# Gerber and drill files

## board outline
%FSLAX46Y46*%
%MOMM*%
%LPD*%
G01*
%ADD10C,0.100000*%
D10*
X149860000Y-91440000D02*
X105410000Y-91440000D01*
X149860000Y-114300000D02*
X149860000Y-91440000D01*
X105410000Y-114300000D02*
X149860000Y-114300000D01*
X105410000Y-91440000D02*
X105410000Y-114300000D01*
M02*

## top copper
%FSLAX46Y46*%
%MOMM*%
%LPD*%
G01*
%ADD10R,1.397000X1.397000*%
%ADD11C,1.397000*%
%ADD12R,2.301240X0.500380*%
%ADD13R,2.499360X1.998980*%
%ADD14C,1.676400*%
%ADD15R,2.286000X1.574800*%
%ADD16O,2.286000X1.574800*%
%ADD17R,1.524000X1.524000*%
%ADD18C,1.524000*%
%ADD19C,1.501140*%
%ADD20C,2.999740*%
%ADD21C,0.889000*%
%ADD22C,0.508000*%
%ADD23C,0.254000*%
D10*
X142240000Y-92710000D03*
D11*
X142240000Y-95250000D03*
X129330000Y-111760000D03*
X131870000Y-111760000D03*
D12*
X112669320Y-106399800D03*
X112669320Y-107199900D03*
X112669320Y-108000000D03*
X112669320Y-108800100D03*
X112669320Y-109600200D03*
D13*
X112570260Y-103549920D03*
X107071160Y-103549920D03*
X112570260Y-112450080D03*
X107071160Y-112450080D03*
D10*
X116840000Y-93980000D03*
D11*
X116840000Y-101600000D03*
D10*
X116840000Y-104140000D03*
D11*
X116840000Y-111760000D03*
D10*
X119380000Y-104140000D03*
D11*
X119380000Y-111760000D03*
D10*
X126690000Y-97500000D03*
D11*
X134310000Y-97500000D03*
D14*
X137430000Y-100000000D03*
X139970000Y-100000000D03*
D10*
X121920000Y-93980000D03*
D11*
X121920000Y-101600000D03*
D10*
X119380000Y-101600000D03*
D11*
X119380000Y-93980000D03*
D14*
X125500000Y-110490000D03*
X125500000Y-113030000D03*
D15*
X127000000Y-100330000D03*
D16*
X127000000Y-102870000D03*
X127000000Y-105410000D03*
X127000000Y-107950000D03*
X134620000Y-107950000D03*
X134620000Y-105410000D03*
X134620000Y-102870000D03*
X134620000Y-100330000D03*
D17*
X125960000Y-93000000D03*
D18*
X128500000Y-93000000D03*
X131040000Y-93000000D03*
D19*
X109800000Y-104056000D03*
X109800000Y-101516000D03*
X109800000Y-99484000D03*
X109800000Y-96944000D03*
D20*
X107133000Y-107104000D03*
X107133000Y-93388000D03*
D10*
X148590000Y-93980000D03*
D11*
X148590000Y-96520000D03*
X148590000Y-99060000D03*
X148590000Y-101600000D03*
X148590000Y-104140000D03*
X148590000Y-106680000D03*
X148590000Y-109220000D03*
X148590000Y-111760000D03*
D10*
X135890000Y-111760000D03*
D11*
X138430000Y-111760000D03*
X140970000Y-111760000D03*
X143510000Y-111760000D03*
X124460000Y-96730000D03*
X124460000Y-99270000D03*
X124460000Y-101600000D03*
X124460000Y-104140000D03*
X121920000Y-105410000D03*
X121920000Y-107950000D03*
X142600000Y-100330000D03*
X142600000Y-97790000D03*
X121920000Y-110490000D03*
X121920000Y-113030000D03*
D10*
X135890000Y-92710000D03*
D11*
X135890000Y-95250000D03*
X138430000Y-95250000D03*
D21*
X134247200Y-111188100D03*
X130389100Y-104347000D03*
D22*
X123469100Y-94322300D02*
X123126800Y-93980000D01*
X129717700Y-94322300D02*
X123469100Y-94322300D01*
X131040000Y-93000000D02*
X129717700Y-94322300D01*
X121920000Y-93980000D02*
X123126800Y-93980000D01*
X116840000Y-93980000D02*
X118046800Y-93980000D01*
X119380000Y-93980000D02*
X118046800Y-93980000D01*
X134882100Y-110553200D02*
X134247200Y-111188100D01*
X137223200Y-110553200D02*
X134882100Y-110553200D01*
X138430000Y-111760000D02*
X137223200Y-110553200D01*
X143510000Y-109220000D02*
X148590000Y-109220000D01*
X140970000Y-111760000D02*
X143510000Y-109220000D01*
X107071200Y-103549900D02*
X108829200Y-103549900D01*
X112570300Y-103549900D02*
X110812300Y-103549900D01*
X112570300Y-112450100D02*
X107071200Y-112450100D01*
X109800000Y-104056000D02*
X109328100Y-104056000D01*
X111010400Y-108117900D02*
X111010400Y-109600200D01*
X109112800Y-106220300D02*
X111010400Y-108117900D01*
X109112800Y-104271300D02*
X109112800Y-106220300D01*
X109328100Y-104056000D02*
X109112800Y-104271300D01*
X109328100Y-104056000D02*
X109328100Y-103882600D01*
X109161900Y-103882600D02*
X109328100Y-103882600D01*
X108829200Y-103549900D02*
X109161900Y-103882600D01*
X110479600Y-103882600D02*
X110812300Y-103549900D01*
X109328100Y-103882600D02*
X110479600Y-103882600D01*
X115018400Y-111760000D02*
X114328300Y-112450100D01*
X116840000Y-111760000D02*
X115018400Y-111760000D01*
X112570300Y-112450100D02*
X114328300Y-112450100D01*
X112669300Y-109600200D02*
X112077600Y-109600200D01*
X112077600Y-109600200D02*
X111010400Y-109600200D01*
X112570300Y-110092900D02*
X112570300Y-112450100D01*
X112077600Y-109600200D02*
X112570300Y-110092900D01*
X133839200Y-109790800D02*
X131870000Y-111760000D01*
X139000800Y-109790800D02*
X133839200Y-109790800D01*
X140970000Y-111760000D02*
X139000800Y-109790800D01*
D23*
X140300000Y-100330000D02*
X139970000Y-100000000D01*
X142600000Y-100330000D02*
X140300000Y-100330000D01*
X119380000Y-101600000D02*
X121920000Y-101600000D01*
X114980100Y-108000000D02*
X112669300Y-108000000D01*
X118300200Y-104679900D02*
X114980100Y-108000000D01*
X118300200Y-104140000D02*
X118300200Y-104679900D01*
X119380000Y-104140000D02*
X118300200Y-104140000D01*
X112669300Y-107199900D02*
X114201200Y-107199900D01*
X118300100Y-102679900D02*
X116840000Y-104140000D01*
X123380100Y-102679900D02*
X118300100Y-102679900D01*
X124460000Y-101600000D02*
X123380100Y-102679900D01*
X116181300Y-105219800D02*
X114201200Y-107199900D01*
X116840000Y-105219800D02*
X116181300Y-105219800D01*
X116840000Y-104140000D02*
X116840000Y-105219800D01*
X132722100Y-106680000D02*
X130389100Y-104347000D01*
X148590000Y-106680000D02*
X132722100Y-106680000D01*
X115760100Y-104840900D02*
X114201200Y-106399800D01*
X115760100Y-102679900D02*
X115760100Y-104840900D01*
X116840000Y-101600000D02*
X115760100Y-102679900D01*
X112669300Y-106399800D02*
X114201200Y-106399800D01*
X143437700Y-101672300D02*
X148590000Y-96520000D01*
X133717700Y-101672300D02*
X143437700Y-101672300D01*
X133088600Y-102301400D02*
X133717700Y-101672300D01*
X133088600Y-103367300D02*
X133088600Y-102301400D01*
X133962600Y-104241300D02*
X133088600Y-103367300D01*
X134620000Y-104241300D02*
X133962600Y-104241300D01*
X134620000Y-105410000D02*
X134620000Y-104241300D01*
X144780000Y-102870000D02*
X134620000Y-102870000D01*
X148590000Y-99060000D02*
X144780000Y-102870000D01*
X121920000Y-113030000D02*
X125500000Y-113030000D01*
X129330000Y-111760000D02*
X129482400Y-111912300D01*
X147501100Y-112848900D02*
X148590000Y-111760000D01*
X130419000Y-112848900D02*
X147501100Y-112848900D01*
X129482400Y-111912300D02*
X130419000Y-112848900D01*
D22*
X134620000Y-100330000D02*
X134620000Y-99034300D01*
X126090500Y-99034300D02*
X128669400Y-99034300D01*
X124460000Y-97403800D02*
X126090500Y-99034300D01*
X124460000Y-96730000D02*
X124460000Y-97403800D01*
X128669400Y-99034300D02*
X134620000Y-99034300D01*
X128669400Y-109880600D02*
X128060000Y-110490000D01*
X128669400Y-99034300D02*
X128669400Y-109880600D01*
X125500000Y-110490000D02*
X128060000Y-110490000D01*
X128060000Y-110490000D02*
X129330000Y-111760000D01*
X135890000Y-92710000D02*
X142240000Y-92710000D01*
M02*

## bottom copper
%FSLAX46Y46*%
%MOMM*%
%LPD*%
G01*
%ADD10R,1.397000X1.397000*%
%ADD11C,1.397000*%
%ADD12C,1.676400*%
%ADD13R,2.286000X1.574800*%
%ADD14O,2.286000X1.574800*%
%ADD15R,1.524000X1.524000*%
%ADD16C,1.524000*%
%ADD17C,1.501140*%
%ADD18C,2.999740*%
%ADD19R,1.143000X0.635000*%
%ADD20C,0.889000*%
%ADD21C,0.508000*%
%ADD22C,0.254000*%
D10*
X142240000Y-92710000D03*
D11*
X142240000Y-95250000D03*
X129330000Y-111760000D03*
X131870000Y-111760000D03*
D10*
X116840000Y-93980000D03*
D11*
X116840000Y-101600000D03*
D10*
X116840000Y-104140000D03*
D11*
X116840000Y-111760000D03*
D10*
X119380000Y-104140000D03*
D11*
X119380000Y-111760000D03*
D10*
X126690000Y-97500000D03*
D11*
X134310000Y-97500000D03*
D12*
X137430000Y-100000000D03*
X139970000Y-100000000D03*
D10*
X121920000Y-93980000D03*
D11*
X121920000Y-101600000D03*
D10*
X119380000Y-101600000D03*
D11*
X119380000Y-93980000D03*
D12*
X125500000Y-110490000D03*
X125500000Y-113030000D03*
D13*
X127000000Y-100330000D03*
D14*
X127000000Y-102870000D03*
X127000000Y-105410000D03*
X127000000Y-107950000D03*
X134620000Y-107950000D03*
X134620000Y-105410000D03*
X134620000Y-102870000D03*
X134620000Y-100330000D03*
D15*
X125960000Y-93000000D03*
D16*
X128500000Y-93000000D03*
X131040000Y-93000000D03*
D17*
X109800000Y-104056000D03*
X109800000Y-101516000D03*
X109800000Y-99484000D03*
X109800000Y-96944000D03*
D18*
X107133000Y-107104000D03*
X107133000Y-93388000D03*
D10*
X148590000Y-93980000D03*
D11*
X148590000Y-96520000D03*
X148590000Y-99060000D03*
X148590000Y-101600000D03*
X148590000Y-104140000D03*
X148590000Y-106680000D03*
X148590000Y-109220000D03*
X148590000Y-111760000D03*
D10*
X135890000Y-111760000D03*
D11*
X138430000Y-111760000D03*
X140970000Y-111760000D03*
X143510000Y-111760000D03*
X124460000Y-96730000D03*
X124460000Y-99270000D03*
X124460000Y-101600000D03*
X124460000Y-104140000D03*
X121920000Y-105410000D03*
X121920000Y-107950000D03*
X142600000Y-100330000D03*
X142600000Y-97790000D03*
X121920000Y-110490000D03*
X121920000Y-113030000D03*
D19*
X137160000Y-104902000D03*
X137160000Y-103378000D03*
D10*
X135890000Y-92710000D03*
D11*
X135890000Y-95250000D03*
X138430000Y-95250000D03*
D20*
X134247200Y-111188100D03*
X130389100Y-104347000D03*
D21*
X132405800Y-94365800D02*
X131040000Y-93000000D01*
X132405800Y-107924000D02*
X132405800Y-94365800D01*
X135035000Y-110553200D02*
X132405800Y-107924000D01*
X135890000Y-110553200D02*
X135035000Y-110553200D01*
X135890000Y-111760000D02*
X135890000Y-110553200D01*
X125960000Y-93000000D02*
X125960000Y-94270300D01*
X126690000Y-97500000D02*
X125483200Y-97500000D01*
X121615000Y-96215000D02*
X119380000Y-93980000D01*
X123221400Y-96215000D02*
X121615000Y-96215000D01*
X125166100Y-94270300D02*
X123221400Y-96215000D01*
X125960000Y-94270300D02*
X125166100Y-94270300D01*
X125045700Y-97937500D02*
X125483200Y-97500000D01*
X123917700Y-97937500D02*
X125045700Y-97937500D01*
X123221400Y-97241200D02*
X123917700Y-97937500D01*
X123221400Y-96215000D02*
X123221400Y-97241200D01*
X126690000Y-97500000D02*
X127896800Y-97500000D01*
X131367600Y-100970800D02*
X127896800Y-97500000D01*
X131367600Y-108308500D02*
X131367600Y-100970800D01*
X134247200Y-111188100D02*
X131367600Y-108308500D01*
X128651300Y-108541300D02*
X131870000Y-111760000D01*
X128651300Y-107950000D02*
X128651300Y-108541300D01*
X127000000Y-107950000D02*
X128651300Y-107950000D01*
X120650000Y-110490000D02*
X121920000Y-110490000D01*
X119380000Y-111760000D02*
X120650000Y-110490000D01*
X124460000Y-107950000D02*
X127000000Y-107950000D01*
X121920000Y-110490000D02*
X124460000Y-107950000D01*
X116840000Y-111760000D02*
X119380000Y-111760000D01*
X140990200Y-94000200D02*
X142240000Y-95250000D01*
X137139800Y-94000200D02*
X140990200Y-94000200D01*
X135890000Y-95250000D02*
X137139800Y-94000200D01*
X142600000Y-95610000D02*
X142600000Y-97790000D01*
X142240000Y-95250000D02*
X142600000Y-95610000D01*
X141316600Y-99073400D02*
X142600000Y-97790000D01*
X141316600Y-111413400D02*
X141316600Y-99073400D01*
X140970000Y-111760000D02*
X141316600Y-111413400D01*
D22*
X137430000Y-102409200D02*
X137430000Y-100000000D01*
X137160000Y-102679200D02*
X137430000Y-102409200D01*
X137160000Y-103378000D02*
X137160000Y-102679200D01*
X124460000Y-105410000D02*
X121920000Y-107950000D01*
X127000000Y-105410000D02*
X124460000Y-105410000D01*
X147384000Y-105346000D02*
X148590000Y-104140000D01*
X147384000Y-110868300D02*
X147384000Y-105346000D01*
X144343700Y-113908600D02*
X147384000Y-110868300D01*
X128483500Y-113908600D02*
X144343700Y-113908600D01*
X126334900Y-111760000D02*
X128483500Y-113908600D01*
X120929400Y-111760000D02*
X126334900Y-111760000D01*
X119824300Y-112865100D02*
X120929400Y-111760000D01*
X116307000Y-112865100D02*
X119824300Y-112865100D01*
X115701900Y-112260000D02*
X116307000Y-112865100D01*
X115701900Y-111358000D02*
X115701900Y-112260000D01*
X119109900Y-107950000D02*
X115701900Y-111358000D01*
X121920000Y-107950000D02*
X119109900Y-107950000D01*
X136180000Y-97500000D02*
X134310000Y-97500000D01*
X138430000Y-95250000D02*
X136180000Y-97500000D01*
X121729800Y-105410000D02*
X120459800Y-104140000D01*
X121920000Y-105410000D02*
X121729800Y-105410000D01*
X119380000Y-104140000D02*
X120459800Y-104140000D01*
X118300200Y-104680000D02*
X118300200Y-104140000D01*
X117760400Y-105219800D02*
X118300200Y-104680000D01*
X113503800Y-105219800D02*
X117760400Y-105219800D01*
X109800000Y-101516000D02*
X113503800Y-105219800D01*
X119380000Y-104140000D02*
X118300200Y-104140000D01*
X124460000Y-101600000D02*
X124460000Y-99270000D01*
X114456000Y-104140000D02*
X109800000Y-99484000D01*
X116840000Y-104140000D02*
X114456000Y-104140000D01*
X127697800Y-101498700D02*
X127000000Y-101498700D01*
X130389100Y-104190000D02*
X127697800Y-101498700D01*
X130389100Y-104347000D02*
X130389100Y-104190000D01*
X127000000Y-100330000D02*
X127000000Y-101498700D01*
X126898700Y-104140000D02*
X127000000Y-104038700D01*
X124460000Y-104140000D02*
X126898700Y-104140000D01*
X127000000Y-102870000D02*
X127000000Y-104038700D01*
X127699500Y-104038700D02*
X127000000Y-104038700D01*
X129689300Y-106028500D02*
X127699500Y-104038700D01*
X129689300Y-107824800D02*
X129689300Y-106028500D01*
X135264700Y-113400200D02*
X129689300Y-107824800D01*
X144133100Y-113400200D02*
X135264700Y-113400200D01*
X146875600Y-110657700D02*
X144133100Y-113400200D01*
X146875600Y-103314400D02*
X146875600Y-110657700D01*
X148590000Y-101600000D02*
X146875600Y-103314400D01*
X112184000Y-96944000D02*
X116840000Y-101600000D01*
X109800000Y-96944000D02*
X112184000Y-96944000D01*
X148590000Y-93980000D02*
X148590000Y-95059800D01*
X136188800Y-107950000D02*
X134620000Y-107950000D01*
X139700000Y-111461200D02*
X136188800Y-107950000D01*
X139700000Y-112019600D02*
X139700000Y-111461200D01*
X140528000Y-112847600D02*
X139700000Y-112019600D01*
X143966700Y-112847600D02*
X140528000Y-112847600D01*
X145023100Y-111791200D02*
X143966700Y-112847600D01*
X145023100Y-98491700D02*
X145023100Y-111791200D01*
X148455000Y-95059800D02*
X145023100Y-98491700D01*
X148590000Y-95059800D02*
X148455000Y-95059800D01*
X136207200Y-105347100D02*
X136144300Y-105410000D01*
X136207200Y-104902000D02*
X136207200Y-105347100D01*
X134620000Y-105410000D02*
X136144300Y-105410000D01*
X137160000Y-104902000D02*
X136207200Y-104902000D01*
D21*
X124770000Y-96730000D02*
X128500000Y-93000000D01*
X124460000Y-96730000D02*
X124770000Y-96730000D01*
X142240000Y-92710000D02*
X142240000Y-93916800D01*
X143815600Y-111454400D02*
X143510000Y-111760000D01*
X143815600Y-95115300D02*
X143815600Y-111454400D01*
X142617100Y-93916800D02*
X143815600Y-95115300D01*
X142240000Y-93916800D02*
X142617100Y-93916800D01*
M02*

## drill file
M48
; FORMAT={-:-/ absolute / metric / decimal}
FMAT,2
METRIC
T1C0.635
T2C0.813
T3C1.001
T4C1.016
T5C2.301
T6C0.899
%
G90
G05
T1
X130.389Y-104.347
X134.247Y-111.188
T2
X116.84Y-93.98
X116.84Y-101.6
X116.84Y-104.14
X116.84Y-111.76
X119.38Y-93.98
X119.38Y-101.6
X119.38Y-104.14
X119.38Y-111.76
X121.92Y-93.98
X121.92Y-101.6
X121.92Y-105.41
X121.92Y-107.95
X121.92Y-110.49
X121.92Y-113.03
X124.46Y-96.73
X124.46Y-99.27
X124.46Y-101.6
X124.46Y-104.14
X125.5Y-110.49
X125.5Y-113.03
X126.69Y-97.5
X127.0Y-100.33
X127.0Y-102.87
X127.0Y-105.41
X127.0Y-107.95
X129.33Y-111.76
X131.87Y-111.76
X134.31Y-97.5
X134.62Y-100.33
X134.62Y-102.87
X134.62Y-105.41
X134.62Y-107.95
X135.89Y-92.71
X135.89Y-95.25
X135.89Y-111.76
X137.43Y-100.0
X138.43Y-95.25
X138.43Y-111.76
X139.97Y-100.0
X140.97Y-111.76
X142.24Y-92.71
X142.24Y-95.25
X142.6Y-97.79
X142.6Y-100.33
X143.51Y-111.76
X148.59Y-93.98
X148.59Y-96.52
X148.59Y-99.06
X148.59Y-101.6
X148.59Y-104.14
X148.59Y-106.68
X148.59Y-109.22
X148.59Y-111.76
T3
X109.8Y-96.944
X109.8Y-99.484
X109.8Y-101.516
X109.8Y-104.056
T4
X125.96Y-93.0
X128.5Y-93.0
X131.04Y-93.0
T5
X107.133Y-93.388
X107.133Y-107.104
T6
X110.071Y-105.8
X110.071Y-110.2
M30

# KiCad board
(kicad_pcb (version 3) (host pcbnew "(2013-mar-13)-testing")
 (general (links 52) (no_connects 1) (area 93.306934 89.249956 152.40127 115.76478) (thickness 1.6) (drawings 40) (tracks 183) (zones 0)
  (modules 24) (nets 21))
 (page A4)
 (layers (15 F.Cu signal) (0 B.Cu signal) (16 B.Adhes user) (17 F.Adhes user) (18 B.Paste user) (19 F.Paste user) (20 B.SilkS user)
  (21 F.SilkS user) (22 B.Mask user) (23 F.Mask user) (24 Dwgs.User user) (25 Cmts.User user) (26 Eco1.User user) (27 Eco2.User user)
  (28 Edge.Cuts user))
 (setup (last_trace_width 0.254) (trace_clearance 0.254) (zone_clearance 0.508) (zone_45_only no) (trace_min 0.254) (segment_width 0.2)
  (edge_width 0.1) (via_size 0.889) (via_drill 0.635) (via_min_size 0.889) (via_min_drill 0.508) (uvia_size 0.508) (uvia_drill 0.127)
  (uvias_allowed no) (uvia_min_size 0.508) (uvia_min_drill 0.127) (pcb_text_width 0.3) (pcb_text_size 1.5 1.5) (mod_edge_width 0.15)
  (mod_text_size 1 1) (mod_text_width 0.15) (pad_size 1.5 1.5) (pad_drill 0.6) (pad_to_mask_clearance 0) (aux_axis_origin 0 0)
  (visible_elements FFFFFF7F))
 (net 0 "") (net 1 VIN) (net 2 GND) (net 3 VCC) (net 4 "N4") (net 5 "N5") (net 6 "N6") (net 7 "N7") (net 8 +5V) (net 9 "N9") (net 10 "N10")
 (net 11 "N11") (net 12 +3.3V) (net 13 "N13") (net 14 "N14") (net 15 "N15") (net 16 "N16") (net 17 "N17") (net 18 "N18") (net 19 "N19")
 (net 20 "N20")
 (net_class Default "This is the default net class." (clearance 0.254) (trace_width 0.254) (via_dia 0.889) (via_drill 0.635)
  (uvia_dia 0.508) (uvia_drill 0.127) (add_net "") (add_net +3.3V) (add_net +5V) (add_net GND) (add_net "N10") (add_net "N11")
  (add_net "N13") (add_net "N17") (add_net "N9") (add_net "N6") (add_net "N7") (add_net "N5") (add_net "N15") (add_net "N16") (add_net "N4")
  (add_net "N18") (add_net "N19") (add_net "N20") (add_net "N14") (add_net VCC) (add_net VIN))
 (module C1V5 (layer F.Cu) (at 142.24 93.98 270)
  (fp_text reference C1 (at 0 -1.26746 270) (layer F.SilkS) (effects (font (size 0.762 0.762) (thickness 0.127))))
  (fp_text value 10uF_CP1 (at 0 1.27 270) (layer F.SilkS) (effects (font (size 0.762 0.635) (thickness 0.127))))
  (pad 1 thru_hole rect (at -1.27 0 270) (size 1.397 1.397) (drill 0.8128) (layers *.Cu *.Mask F.SilkS) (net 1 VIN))
  (pad 2 thru_hole circle (at 1.27 0 270) (size 1.397 1.397) (drill 0.8128) (layers *.Cu *.Mask F.SilkS) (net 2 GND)))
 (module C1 (layer F.Cu) (at 130.6 111.76)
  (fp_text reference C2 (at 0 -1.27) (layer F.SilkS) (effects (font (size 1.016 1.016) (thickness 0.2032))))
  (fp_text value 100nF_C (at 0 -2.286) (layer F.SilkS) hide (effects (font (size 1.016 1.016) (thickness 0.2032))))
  (pad 1 thru_hole circle (at -1.27 0) (size 1.397 1.397) (drill 0.8128) (layers *.Cu *.Mask F.SilkS) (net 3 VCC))
  (pad 2 thru_hole circle (at 1.27 0) (size 1.397 1.397) (drill 0.8128) (layers *.Cu *.Mask F.SilkS) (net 2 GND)))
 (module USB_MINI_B (layer F.Cu) (at 109.22 108)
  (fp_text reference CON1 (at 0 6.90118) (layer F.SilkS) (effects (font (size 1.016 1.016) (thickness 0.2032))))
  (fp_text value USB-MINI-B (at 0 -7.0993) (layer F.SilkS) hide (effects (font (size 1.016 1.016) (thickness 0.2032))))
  (pad 1 smd rect (at 3.44932 -1.6002) (size 2.30124 0.50038) (layers F.Cu F.Paste F.Mask) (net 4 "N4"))
  (pad 2 smd rect (at 3.44932 -0.8001) (size 2.30124 0.50038) (layers F.Cu F.Paste F.Mask) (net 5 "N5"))
  (pad 3 smd rect (at 3.44932 0) (size 2.30124 0.50038) (layers F.Cu F.Paste F.Mask) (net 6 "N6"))
  (pad 4 smd rect (at 3.44932 0.8001) (size 2.30124 0.50038) (layers F.Cu F.Paste F.Mask) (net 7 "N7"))
  (pad 5 smd rect (at 3.44932 1.6002) (size 2.30124 0.50038) (layers F.Cu F.Paste F.Mask) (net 2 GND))
  (pad 6 smd rect (at 3.35026 -4.45008) (size 2.49936 1.99898) (layers F.Cu F.Paste F.Mask) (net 2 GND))
  (pad 7 smd rect (at -2.14884 -4.45008) (size 2.49936 1.99898) (layers F.Cu F.Paste F.Mask) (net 2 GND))
  (pad 8 smd rect (at 3.35026 4.45008) (size 2.49936 1.99898) (layers F.Cu F.Paste F.Mask) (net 2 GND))
  (pad 9 smd rect (at -2.14884 4.45008) (size 2.49936 1.99898) (layers F.Cu F.Paste F.Mask) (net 2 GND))
  (pad "" np_thru_hole circle (at 0.8509 -2.19964) (size 0.89916 0.89916) (drill 0.89916) (layers *.Cu *.Mask F.SilkS))
  (pad 2 np_thru_hole circle (at 0.8509 2.19964) (size 0.89916 0.89916) (drill 0.89916) (layers *.Cu *.Mask F.SilkS) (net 5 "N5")))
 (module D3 (layer F.Cu) (at 116.84 97.79 90)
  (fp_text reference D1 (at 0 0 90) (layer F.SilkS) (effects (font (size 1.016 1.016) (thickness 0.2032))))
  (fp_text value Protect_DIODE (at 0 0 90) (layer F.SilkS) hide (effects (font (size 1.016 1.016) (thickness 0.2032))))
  (pad 2 thru_hole rect (at 3.81 0 90) (size 1.397 1.397) (drill 0.8128) (layers *.Cu *.Mask F.SilkS) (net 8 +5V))
  (pad 1 thru_hole circle (at -3.81 0 90) (size 1.397 1.397) (drill 0.8128) (layers *.Cu *.Mask F.SilkS) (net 4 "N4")))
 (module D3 (layer F.Cu) (at 116.84 107.95 90)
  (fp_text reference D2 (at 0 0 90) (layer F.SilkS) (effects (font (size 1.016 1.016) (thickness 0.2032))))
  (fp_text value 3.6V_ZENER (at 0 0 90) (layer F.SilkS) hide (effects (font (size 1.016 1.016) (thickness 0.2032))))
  (pad 2 thru_hole rect (at 3.81 0 90) (size 1.397 1.397) (drill 0.8128) (layers *.Cu *.Mask F.SilkS) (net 5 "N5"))
  (pad 1 thru_hole circle (at -3.81 0 90) (size 1.397 1.397) (drill 0.8128) (layers *.Cu *.Mask F.SilkS) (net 2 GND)))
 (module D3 (layer F.Cu) (at 119.38 107.95 90)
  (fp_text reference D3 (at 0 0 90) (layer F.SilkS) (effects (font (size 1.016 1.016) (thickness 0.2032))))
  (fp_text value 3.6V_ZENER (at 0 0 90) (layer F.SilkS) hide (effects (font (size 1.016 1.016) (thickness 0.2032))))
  (pad 2 thru_hole rect (at 3.81 0 90) (size 1.397 1.397) (drill 0.8128) (layers *.Cu *.Mask F.SilkS) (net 6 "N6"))
  (pad 1 thru_hole circle (at -3.81 0 90) (size 1.397 1.397) (drill 0.8128) (layers *.Cu *.Mask F.SilkS) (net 2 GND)))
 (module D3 (layer F.Cu) (at 130.5 97.5 180)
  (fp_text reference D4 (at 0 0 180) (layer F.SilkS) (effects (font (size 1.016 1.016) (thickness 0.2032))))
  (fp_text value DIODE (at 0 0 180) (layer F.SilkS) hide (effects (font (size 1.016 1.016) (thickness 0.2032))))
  (pad 2 thru_hole rect (at 3.81 0 180) (size 1.397 1.397) (drill 0.8128) (layers *.Cu *.Mask F.SilkS) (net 8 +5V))
  (pad 1 thru_hole circle (at -3.81 0 180) (size 1.397 1.397) (drill 0.8128) (layers *.Cu *.Mask F.SilkS) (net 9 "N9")))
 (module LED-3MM (layer F.Cu) (at 138.7 100)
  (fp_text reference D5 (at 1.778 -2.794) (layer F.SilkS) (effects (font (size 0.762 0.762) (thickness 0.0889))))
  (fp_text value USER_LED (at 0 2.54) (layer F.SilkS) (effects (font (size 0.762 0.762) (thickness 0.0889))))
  (pad 1 thru_hole circle (at -1.27 0) (size 1.6764 1.6764) (drill 0.8128) (layers *.Cu *.Mask F.SilkS) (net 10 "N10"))
  (pad 2 thru_hole circle (at 1.27 0) (size 1.6764 1.6764) (drill 0.8128) (layers *.Cu *.Mask F.SilkS) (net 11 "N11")))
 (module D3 (layer F.Cu) (at 121.92 97.79 90)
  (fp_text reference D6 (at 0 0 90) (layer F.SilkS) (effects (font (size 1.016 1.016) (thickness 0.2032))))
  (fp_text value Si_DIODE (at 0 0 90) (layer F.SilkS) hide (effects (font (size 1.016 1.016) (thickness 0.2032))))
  (pad 2 thru_hole rect (at 3.81 0 90) (size 1.397 1.397) (drill 0.8128) (layers *.Cu *.Mask F.SilkS) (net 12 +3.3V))
  (pad 1 thru_hole circle (at -3.81 0 90) (size 1.397 1.397) (drill 0.8128) (layers *.Cu *.Mask F.SilkS) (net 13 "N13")))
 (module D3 (layer F.Cu) (at 119.38 97.79 270)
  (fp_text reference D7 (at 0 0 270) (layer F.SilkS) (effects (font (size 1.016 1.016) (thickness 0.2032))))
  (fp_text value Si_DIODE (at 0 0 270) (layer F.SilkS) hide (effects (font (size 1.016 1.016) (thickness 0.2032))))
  (pad 2 thru_hole rect (at 3.81 0 270) (size 1.397 1.397) (drill 0.8128) (layers *.Cu *.Mask F.SilkS) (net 13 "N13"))
  (pad 1 thru_hole circle (at -3.81 0 270) (size 1.397 1.397) (drill 0.8128) (layers *.Cu *.Mask F.SilkS) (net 8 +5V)))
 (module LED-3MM (layer F.Cu) (at 125.5 111.76 270)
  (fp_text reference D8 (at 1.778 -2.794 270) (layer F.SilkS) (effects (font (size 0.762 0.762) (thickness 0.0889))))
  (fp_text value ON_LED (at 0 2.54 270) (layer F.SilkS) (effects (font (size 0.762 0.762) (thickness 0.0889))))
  (pad 1 thru_hole circle (at -1.27 0 270) (size 1.6764 1.6764) (drill 0.8128) (layers *.Cu *.Mask F.SilkS) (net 3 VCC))
  (pad 2 thru_hole circle (at 1.27 0 270) (size 1.6764 1.6764) (drill 0.8128) (layers *.Cu *.Mask F.SilkS) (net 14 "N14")))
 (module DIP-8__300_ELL (layer F.Cu) (at 130.81 104.14 270)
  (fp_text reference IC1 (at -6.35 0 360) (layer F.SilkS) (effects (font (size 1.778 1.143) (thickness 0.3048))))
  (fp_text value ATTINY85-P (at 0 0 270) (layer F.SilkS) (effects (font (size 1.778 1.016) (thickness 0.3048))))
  (pad 1 thru_hole rect (at -3.81 3.81 270) (size 1.5748 2.286) (drill 0.8128) (layers *.Cu *.Mask F.SilkS) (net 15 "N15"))
  (pad 2 thru_hole oval (at -1.27 3.81 270) (size 1.5748 2.286) (drill 0.8128) (layers *.Cu *.Mask F.SilkS) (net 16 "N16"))
  (pad 3 thru_hole oval (at 1.27 3.81 270) (size 1.5748 2.286) (drill 0.8128) (layers *.Cu *.Mask F.SilkS) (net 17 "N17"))
  (pad 4 thru_hole oval (at 3.81 3.81 270) (size 1.5748 2.286) (drill 0.8128) (layers *.Cu *.Mask F.SilkS) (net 2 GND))
  (pad 5 thru_hole oval (at 3.81 -3.81 270) (size 1.5748 2.286) (drill 0.8128) (layers *.Cu *.Mask F.SilkS) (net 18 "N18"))
  (pad 6 thru_hole oval (at 1.27 -3.81 270) (size 1.5748 2.286) (drill 0.8128) (layers *.Cu *.Mask F.SilkS) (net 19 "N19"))
  (pad 7 thru_hole oval (at -1.27 -3.81 270) (size 1.5748 2.286) (drill 0.8128) (layers *.Cu *.Mask F.SilkS) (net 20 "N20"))
  (pad 8 thru_hole oval (at -3.81 -3.81 270) (size 1.5748 2.286) (drill 0.8128) (layers *.Cu *.Mask F.SilkS) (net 3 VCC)))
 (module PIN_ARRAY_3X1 (layer F.Cu) (at 128.5 93)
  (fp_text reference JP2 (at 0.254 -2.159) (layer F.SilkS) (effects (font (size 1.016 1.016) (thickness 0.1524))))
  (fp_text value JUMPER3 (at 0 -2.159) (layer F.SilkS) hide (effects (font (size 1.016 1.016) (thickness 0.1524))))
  (pad 1 thru_hole rect (at -2.54 0) (size 1.524 1.524) (drill 1.016) (layers *.Cu *.Mask F.SilkS) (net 8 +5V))
  (pad 2 thru_hole circle (at 0 0) (size 1.524 1.524) (drill 1.016) (layers *.Cu *.Mask F.SilkS) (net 3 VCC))
  (pad 3 thru_hole circle (at 2.54 0) (size 1.524 1.524) (drill 1.016) (layers *.Cu *.Mask F.SilkS) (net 12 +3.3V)))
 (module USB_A (layer F.Cu) (at 109.8 100.5 180)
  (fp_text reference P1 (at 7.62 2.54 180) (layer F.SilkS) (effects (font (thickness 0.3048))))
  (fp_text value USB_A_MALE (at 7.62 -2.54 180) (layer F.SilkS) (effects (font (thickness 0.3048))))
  (pad 4 thru_hole circle (at 0 -3.556 180) (size 1.50114 1.50114) (drill 1.00076) (layers *.Cu *.Mask F.SilkS) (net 2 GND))
  (pad 3 thru_hole circle (at 0 -1.016 180) (size 1.50114 1.50114) (drill 1.00076) (layers *.Cu *.Mask F.SilkS) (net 6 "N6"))
  (pad 2 thru_hole circle (at 0 1.016 180) (size 1.50114 1.50114) (drill 1.00076) (layers *.Cu *.Mask F.SilkS) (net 5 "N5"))
  (pad 1 thru_hole circle (at 0 3.556 180) (size 1.50114 1.50114) (drill 1.00076) (layers *.Cu *.Mask F.SilkS) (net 4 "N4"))
  (pad 5 thru_hole circle (at 2.667 -6.604 180) (size 2.99974 2.99974) (drill 2.30124) (layers *.Cu *.Mask F.SilkS))
  (pad 6 thru_hole circle (at 2.667 7.112 180) (size 2.99974 2.99974) (drill 2.30124) (layers *.Cu *.Mask F.SilkS)))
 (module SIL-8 (layer F.Cu) (at 148.59 102.87 270)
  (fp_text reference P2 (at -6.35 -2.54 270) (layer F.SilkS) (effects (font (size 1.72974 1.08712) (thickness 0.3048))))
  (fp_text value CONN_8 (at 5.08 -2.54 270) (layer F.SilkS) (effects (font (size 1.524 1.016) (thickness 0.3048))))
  (pad 1 thru_hole rect (at -8.89 0 270) (size 1.397 1.397) (drill 0.8128) (layers *.Cu *.Mask F.SilkS) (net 18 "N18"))
  (pad 2 thru_hole circle (at -6.35 0 270) (size 1.397 1.397) (drill 0.8128) (layers *.Cu *.Mask F.SilkS) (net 19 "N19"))
  (pad 3 thru_hole circle (at -3.81 0 270) (size 1.397 1.397) (drill 0.8128) (layers *.Cu *.Mask F.SilkS) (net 20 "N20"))
  (pad 4 thru_hole circle (at -1.27 0 270) (size 1.397 1.397) (drill 0.8128) (layers *.Cu *.Mask F.SilkS) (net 16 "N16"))
  (pad 5 thru_hole circle (at 1.27 0 270) (size 1.397 1.397) (drill 0.8128) (layers *.Cu *.Mask F.SilkS) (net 17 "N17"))
  (pad 6 thru_hole circle (at 3.81 0 270) (size 1.397 1.397) (drill 0.8128) (layers *.Cu *.Mask F.SilkS) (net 15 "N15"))
  (pad 7 thru_hole circle (at 6.35 0 270) (size 1.397 1.397) (drill 0.8128) (layers *.Cu *.Mask F.SilkS) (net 2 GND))
  (pad 8 thru_hole circle (at 8.89 0 270) (size 1.397 1.397) (drill 0.8128) (layers *.Cu *.Mask F.SilkS) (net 3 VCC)))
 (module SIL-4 (layer F.Cu) (at 139.7 111.76)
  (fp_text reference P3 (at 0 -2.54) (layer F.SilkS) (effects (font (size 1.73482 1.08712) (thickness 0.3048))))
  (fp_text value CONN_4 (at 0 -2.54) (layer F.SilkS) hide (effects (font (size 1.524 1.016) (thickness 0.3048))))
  (pad 1 thru_hole rect (at -3.81 0) (size 1.397 1.397) (drill 0.8128) (layers *.Cu *.Mask F.SilkS) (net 12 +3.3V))
  (pad 2 thru_hole circle (at -1.27 0) (size 1.397 1.397) (drill 0.8128) (layers *.Cu *.Mask F.SilkS) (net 8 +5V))
  (pad 3 thru_hole circle (at 1.27 0) (size 1.397 1.397) (drill 0.8128) (layers *.Cu *.Mask F.SilkS) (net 2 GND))
  (pad 4 thru_hole circle (at 3.81 0) (size 1.397 1.397) (drill 0.8128) (layers *.Cu *.Mask F.SilkS) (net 1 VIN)))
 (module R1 (layer F.Cu) (at 124.46 98 270) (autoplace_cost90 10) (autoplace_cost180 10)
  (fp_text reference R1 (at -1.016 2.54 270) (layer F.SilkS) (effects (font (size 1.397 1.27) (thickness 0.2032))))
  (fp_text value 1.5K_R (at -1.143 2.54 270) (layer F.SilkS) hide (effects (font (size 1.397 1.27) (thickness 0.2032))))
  (pad 1 thru_hole circle (at -1.27 0 270) (size 1.397 1.397) (drill 0.8128) (layers *.Cu *.Mask F.SilkS) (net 3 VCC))
  (pad 2 thru_hole circle (at 1.27 0 270) (size 1.397 1.397) (drill 0.8128) (layers *.Cu *.Mask F.SilkS) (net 5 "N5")))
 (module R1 (layer F.Cu) (at 124.46 102.87 270) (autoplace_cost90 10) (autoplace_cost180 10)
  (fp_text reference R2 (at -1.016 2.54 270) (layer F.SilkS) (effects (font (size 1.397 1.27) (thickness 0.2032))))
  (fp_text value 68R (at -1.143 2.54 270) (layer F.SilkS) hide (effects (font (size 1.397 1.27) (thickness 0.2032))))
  (pad 1 thru_hole circle (at -1.27 0 270) (size 1.397 1.397) (drill 0.8128) (layers *.Cu *.Mask F.SilkS) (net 5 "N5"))
  (pad 2 thru_hole circle (at 1.27 0 270) (size 1.397 1.397) (drill 0.8128) (layers *.Cu *.Mask F.SilkS) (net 16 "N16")))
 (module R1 (layer F.Cu) (at 121.92 106.68 270) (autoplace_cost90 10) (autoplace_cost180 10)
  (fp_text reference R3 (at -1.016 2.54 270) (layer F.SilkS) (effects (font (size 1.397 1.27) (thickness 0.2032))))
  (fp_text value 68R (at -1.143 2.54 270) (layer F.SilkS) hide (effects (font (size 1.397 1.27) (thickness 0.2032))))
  (pad 1 thru_hole circle (at -1.27 0 270) (size 1.397 1.397) (drill 0.8128) (layers *.Cu *.Mask F.SilkS) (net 6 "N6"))
  (pad 2 thru_hole circle (at 1.27 0 270) (size 1.397 1.397) (drill 0.8128) (layers *.Cu *.Mask F.SilkS) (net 17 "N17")))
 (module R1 (layer F.Cu) (at 142.6 99.06 90) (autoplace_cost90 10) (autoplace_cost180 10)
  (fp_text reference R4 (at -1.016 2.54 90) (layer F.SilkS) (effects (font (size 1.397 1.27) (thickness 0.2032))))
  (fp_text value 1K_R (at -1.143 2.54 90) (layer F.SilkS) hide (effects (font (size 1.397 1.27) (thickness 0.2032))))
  (pad 1 thru_hole circle (at -1.27 0 90) (size 1.397 1.397) (drill 0.8128) (layers *.Cu *.Mask F.SilkS) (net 11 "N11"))
  (pad 2 thru_hole circle (at 1.27 0 90) (size 1.397 1.397) (drill 0.8128) (layers *.Cu *.Mask F.SilkS) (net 2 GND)))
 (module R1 (layer F.Cu) (at 121.92 111.76 270) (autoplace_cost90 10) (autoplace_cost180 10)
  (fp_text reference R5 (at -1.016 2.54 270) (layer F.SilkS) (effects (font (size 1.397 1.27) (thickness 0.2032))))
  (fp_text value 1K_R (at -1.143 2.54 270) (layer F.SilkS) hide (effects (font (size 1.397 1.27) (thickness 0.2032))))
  (pad 1 thru_hole circle (at -1.27 0 270) (size 1.397 1.397) (drill 0.8128) (layers *.Cu *.Mask F.SilkS) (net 2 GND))
  (pad 2 thru_hole circle (at 1.27 0 270) (size 1.397 1.397) (drill 0.8128) (layers *.Cu *.Mask F.SilkS) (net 14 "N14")))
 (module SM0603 (layer B.Cu) (at 137.16 104.14 90)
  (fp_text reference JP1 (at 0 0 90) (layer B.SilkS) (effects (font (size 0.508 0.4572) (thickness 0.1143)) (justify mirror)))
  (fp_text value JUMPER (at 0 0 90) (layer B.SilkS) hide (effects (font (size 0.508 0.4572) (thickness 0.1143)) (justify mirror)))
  (pad 1 smd rect (at -0.762 0 90) (size 0.635 1.143) (layers B.Cu B.Paste B.Mask) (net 19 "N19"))
  (pad 2 smd rect (at 0.762 0 90) (size 0.635 1.143) (layers B.Cu B.Paste B.Mask) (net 10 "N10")))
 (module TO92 (layer F.Cu) (at 137.16 93.98 90)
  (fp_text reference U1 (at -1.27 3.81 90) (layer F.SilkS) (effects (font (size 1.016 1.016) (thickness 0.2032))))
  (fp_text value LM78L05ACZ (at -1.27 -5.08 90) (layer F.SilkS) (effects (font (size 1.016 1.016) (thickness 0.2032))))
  (pad 1 thru_hole rect (at 1.27 -1.27 90) (size 1.397 1.397) (drill 0.8128) (layers *.Cu *.Mask F.SilkS) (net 1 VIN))
  (pad 2 thru_hole circle (at -1.27 -1.27 90) (size 1.397 1.397) (drill 0.8128) (layers *.Cu *.Mask F.SilkS) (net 2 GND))
  (pad 3 thru_hole circle (at -1.27 1.27 90) (size 1.397 1.397) (drill 0.8128) (layers *.Cu *.Mask F.SilkS) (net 9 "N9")))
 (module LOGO (layer F.Cu) (at 114.3 100.33 90)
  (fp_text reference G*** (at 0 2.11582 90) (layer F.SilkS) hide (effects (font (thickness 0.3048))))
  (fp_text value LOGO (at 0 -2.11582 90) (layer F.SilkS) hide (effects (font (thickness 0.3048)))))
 (gr_line (start 149.86 91.44) (end 105.41 91.44) (angle 90) (layer Edge.Cuts) (width 0.1))
 (gr_line (start 149.86 114.3) (end 149.86 91.44) (angle 90) (layer Edge.Cuts) (width 0.1))
 (gr_line (start 105.41 114.3) (end 149.86 114.3) (angle 90) (layer Edge.Cuts) (width 0.1))
 (gr_line (start 105.41 91.44) (end 105.41 114.3) (angle 90) (layer Edge.Cuts) (width 0.1))
 (segment (start 123.4691 94.3223) (end 123.1268 93.98) (width 0.508) (layer F.Cu) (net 12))
 (segment (start 129.7177 94.3223) (end 123.4691 94.3223) (width 0.508) (layer F.Cu) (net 12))
 (segment (start 131.04 93) (end 129.7177 94.3223) (width 0.508) (layer F.Cu) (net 12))
 (segment (start 121.92 93.98) (end 123.1268 93.98) (width 0.508) (layer F.Cu) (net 12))
 (segment (start 132.4058 94.3658) (end 131.04 93) (width 0.508) (layer B.Cu) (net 12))
 (segment (start 132.4058 107.924) (end 132.4058 94.3658) (width 0.508) (layer B.Cu) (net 12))
 (segment (start 135.035 110.5532) (end 132.4058 107.924) (width 0.508) (layer B.Cu) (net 12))
 (segment (start 135.89 110.5532) (end 135.035 110.5532) (width 0.508) (layer B.Cu) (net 12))
 (segment (start 135.89 111.76) (end 135.89 110.5532) (width 0.508) (layer B.Cu) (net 12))
 (via (at 134.2472 111.1881) (size 0.889) (layers F.Cu B.Cu) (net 8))
 (segment (start 116.84 93.98) (end 118.0468 93.98) (width 0.508) (layer F.Cu) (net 8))
 (segment (start 119.38 93.98) (end 118.0468 93.98) (width 0.508) (layer F.Cu) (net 8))
 (segment (start 125.96 93) (end 125.96 94.2703) (width 0.508) (layer B.Cu) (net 8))
 (segment (start 126.69 97.5) (end 125.4832 97.5) (width 0.508) (layer B.Cu) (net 8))
 (segment (start 121.615 96.215) (end 119.38 93.98) (width 0.508) (layer B.Cu) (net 8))
 (segment (start 123.2214 96.215) (end 121.615 96.215) (width 0.508) (layer B.Cu) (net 8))
 (segment (start 125.1661 94.2703) (end 123.2214 96.215) (width 0.508) (layer B.Cu) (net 8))
 (segment (start 125.96 94.2703) (end 125.1661 94.2703) (width 0.508) (layer B.Cu) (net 8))
 (segment (start 125.0457 97.9375) (end 125.4832 97.5) (width 0.508) (layer B.Cu) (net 8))
 (segment (start 123.9177 97.9375) (end 125.0457 97.9375) (width 0.508) (layer B.Cu) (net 8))
 (segment (start 123.2214 97.2412) (end 123.9177 97.9375) (width 0.508) (layer B.Cu) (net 8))
 (segment (start 123.2214 96.215) (end 123.2214 97.2412) (width 0.508) (layer B.Cu) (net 8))
 (segment (start 126.69 97.5) (end 127.8968 97.5) (width 0.508) (layer B.Cu) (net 8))
 (segment (start 134.8821 110.5532) (end 134.2472 111.1881) (width 0.508) (layer F.Cu) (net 8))
 (segment (start 137.2232 110.5532) (end 134.8821 110.5532) (width 0.508) (layer F.Cu) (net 8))
 (segment (start 138.43 111.76) (end 137.2232 110.5532) (width 0.508) (layer F.Cu) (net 8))
 (segment (start 131.3676 100.9708) (end 127.8968 97.5) (width 0.508) (layer B.Cu) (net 8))
 (segment (start 131.3676 108.3085) (end 131.3676 100.9708) (width 0.508) (layer B.Cu) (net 8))
 (segment (start 134.2472 111.1881) (end 131.3676 108.3085) (width 0.508) (layer B.Cu) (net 8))
 (segment (start 128.6513 108.5413) (end 131.87 111.76) (width 0.508) (layer B.Cu) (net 2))
 (segment (start 128.6513 107.95) (end 128.6513 108.5413) (width 0.508) (layer B.Cu) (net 2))
 (segment (start 127 107.95) (end 128.6513 107.95) (width 0.508) (layer B.Cu) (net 2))
 (segment (start 120.65 110.49) (end 121.92 110.49) (width 0.508) (layer B.Cu) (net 2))
 (segment (start 119.38 111.76) (end 120.65 110.49) (width 0.508) (layer B.Cu) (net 2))
 (segment (start 124.46 107.95) (end 127 107.95) (width 0.508) (layer B.Cu) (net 2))
 (segment (start 121.92 110.49) (end 124.46 107.95) (width 0.508) (layer B.Cu) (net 2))
 (segment (start 116.84 111.76) (end 119.38 111.76) (width 0.508) (layer B.Cu) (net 2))
 (segment (start 143.51 109.22) (end 148.59 109.22) (width 0.508) (layer F.Cu) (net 2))
 (segment (start 140.97 111.76) (end 143.51 109.22) (width 0.508) (layer F.Cu) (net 2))
 (segment (start 140.9902 94.0002) (end 142.24 95.25) (width 0.508) (layer B.Cu) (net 2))
 (segment (start 137.1398 94.0002) (end 140.9902 94.0002) (width 0.508) (layer B.Cu) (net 2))
 (segment (start 135.89 95.25) (end 137.1398 94.0002) (width 0.508) (layer B.Cu) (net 2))
 (segment (start 142.6 95.61) (end 142.6 97.79) (width 0.508) (layer B.Cu) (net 2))
 (segment (start 142.24 95.25) (end 142.6 95.61) (width 0.508) (layer B.Cu) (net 2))
 (segment (start 141.3166 99.0734) (end 142.6 97.79) (width 0.508) (layer B.Cu) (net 2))
 (segment (start 141.3166 111.4134) (end 141.3166 99.0734) (width 0.508) (layer B.Cu) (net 2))
 (segment (start 140.97 111.76) (end 141.3166 111.4134) (width 0.508) (layer B.Cu) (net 2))
 (segment (start 107.0712 103.5499) (end 108.8292 103.5499) (width 0.508) (layer F.Cu) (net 2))
 (segment (start 112.5703 103.5499) (end 110.8123 103.5499) (width 0.508) (layer F.Cu) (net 2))
 (segment (start 112.5703 112.4501) (end 107.0712 112.4501) (width 0.508) (layer F.Cu) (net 2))
 (segment (start 109.8 104.056) (end 109.3281 104.056) (width 0.508) (layer F.Cu) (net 2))
 (segment (start 111.0104 108.1179) (end 111.0104 109.6002) (width 0.508) (layer F.Cu) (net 2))
 (segment (start 109.1128 106.2203) (end 111.0104 108.1179) (width 0.508) (layer F.Cu) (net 2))
 (segment (start 109.1128 104.2713) (end 109.1128 106.2203) (width 0.508) (layer F.Cu) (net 2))
 (segment (start 109.3281 104.056) (end 109.1128 104.2713) (width 0.508) (layer F.Cu) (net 2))
 (segment (start 109.3281 104.056) (end 109.3281 103.8826) (width 0.508) (layer F.Cu) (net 2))
 (segment (start 109.1619 103.8826) (end 109.3281 103.8826) (width 0.508) (layer F.Cu) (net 2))
 (segment (start 108.8292 103.5499) (end 109.1619 103.8826) (width 0.508) (layer F.Cu) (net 2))
 (segment (start 110.4796 103.8826) (end 110.8123 103.5499) (width 0.508) (layer F.Cu) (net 2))
 (segment (start 109.3281 103.8826) (end 110.4796 103.8826) (width 0.508) (layer F.Cu) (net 2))
 (segment (start 115.0184 111.76) (end 114.3283 112.4501) (width 0.508) (layer F.Cu) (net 2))
 (segment (start 116.84 111.76) (end 115.0184 111.76) (width 0.508) (layer F.Cu) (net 2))
 (segment (start 112.5703 112.4501) (end 114.3283 112.4501) (width 0.508) (layer F.Cu) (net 2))
 (segment (start 112.6693 109.6002) (end 112.0776 109.6002) (width 0.508) (layer F.Cu) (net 2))
 (segment (start 112.0776 109.6002) (end 111.0104 109.6002) (width 0.508) (layer F.Cu) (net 2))
 (segment (start 112.5703 110.0929) (end 112.5703 112.4501) (width 0.508) (layer F.Cu) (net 2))
 (segment (start 112.0776 109.6002) (end 112.5703 110.0929) (width 0.508) (layer F.Cu) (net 2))
 (segment (start 133.8392 109.7908) (end 131.87 111.76) (width 0.508) (layer F.Cu) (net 2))
 (segment (start 139.0008 109.7908) (end 133.8392 109.7908) (width 0.508) (layer F.Cu) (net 2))
 (segment (start 140.97 111.76) (end 139.0008 109.7908) (width 0.508) (layer F.Cu) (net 2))
 (segment (start 137.43 102.4092) (end 137.43 100) (width 0.254) (layer B.Cu) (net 10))
 (segment (start 137.16 102.6792) (end 137.43 102.4092) (width 0.254) (layer B.Cu) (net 10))
 (segment (start 137.16 103.378) (end 137.16 102.6792) (width 0.254) (layer B.Cu) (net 10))
 (segment (start 140.3 100.33) (end 139.97 100) (width 0.254) (layer F.Cu) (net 11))
 (segment (start 142.6 100.33) (end 140.3 100.33) (width 0.254) (layer F.Cu) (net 11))
 (segment (start 119.38 101.6) (end 121.92 101.6) (width 0.254) (layer F.Cu) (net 13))
 (segment (start 124.46 105.41) (end 121.92 107.95) (width 0.254) (layer B.Cu) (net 17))
 (segment (start 127 105.41) (end 124.46 105.41) (width 0.254) (layer B.Cu) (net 17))
 (segment (start 147.384 105.346) (end 148.59 104.14) (width 0.254) (layer B.Cu) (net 17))
 (segment (start 147.384 110.8683) (end 147.384 105.346) (width 0.254) (layer B.Cu) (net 17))
 (segment (start 144.3437 113.9086) (end 147.384 110.8683) (width 0.254) (layer B.Cu) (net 17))
 (segment (start 128.4835 113.9086) (end 144.3437 113.9086) (width 0.254) (layer B.Cu) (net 17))
 (segment (start 126.3349 111.76) (end 128.4835 113.9086) (width 0.254) (layer B.Cu) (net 17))
 (segment (start 120.9294 111.76) (end 126.3349 111.76) (width 0.254) (layer B.Cu) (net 17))
 (segment (start 119.8243 112.8651) (end 120.9294 111.76) (width 0.254) (layer B.Cu) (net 17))
 (segment (start 116.307 112.8651) (end 119.8243 112.8651) (width 0.254) (layer B.Cu) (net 17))
 (segment (start 115.7019 112.26) (end 116.307 112.8651) (width 0.254) (layer B.Cu) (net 17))
 (segment (start 115.7019 111.358) (end 115.7019 112.26) (width 0.254) (layer B.Cu) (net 17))
 (segment (start 119.1099 107.95) (end 115.7019 111.358) (width 0.254) (layer B.Cu) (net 17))
 (segment (start 121.92 107.95) (end 119.1099 107.95) (width 0.254) (layer B.Cu) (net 17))
 (segment (start 136.18 97.5) (end 134.31 97.5) (width 0.254) (layer B.Cu) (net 9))
 (segment (start 138.43 95.25) (end 136.18 97.5) (width 0.254) (layer B.Cu) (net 9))
 (segment (start 121.7298 105.41) (end 120.4598 104.14) (width 0.254) (layer B.Cu) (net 6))
 (segment (start 121.92 105.41) (end 121.7298 105.41) (width 0.254) (layer B.Cu) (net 6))
 (segment (start 119.38 104.14) (end 120.4598 104.14) (width 0.254) (layer B.Cu) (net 6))
 (segment (start 118.3002 104.68) (end 118.3002 104.14) (width 0.254) (layer B.Cu) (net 6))
 (segment (start 117.7604 105.2198) (end 118.3002 104.68) (width 0.254) (layer B.Cu) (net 6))
 (segment (start 113.5038 105.2198) (end 117.7604 105.2198) (width 0.254) (layer B.Cu) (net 6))
 (segment (start 109.8 101.516) (end 113.5038 105.2198) (width 0.254) (layer B.Cu) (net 6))
 (segment (start 119.38 104.14) (end 118.3002 104.14) (width 0.254) (layer B.Cu) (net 6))
 (segment (start 114.9801 108) (end 112.6693 108) (width 0.254) (layer F.Cu) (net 6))
 (segment (start 118.3002 104.6799) (end 114.9801 108) (width 0.254) (layer F.Cu) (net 6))
 (segment (start 118.3002 104.14) (end 118.3002 104.6799) (width 0.254) (layer F.Cu) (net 6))
 (segment (start 119.38 104.14) (end 118.3002 104.14) (width 0.254) (layer F.Cu) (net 6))
 (segment (start 124.46 101.6) (end 124.46 99.27) (width 0.254) (layer B.Cu) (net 5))
 (segment (start 112.6693 107.1999) (end 114.2012 107.1999) (width 0.254) (layer F.Cu) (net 5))
 (segment (start 118.3001 102.6799) (end 116.84 104.14) (width 0.254) (layer F.Cu) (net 5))
 (segment (start 123.3801 102.6799) (end 118.3001 102.6799) (width 0.254) (layer F.Cu) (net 5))
 (segment (start 124.46 101.6) (end 123.3801 102.6799) (width 0.254) (layer F.Cu) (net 5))
 (segment (start 116.1813 105.2198) (end 114.2012 107.1999) (width 0.254) (layer F.Cu) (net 5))
 (segment (start 116.84 105.2198) (end 116.1813 105.2198) (width 0.254) (layer F.Cu) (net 5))
 (segment (start 116.84 104.14) (end 116.84 105.2198) (width 0.254) (layer F.Cu) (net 5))
 (segment (start 114.456 104.14) (end 109.8 99.484) (width 0.254) (layer B.Cu) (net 5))
 (segment (start 116.84 104.14) (end 114.456 104.14) (width 0.254) (layer B.Cu) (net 5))
 (via (at 130.3891 104.347) (size 0.889) (layers F.Cu B.Cu) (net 15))
 (segment (start 132.7221 106.68) (end 130.3891 104.347) (width 0.254) (layer F.Cu) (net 15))
 (segment (start 148.59 106.68) (end 132.7221 106.68) (width 0.254) (layer F.Cu) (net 15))
 (segment (start 127.6978 101.4987) (end 127 101.4987) (width 0.254) (layer B.Cu) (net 15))
 (segment (start 130.3891 104.19) (end 127.6978 101.4987) (width 0.254) (layer B.Cu) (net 15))
 (segment (start 130.3891 104.347) (end 130.3891 104.19) (width 0.254) (layer B.Cu) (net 15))
 (segment (start 127 100.33) (end 127 101.4987) (width 0.254) (layer B.Cu) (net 15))
 (segment (start 126.8987 104.14) (end 127 104.0387) (width 0.254) (layer B.Cu) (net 16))
 (segment (start 124.46 104.14) (end 126.8987 104.14) (width 0.254) (layer B.Cu) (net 16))
 (segment (start 127 102.87) (end 127 104.0387) (width 0.254) (layer B.Cu) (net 16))
 (segment (start 127.6995 104.0387) (end 127 104.0387) (width 0.254) (layer B.Cu) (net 16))
 (segment (start 129.6893 106.0285) (end 127.6995 104.0387) (width 0.254) (layer B.Cu) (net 16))
 (segment (start 129.6893 107.8248) (end 129.6893 106.0285) (width 0.254) (layer B.Cu) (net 16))
 (segment (start 135.2647 113.4002) (end 129.6893 107.8248) (width 0.254) (layer B.Cu) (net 16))
 (segment (start 144.1331 113.4002) (end 135.2647 113.4002) (width 0.254) (layer B.Cu) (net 16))
 (segment (start 146.8756 110.6577) (end 144.1331 113.4002) (width 0.254) (layer B.Cu) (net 16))
 (segment (start 146.8756 103.3144) (end 146.8756 110.6577) (width 0.254) (layer B.Cu) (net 16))
 (segment (start 148.59 101.6) (end 146.8756 103.3144) (width 0.254) (layer B.Cu) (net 16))
 (segment (start 112.184 96.944) (end 116.84 101.6) (width 0.254) (layer B.Cu) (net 4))
 (segment (start 109.8 96.944) (end 112.184 96.944) (width 0.254) (layer B.Cu) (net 4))
 (segment (start 115.7601 104.8409) (end 114.2012 106.3998) (width 0.254) (layer F.Cu) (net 4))
 (segment (start 115.7601 102.6799) (end 115.7601 104.8409) (width 0.254) (layer F.Cu) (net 4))
 (segment (start 116.84 101.6) (end 115.7601 102.6799) (width 0.254) (layer F.Cu) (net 4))
 (segment (start 112.6693 106.3998) (end 114.2012 106.3998) (width 0.254) (layer F.Cu) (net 4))
 (segment (start 148.59 93.98) (end 148.59 95.0598) (width 0.254) (layer B.Cu) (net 18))
 (segment (start 136.1888 107.95) (end 134.62 107.95) (width 0.254) (layer B.Cu) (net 18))
 (segment (start 139.7 111.4612) (end 136.1888 107.95) (width 0.254) (layer B.Cu) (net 18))
 (segment (start 139.7 112.0196) (end 139.7 111.4612) (width 0.254) (layer B.Cu) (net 18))
 (segment (start 140.528 112.8476) (end 139.7 112.0196) (width 0.254) (layer B.Cu) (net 18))
 (segment (start 143.9667 112.8476) (end 140.528 112.8476) (width 0.254) (layer B.Cu) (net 18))
 (segment (start 145.0231 111.7912) (end 143.9667 112.8476) (width 0.254) (layer B.Cu) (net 18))
 (segment (start 145.0231 98.4917) (end 145.0231 111.7912) (width 0.254) (layer B.Cu) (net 18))
 (segment (start 148.455 95.0598) (end 145.0231 98.4917) (width 0.254) (layer B.Cu) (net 18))
 (segment (start 148.59 95.0598) (end 148.455 95.0598) (width 0.254) (layer B.Cu) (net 18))
 (segment (start 136.2072 105.3471) (end 136.1443 105.41) (width 0.254) (layer B.Cu) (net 19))
 (segment (start 136.2072 104.902) (end 136.2072 105.3471) (width 0.254) (layer B.Cu) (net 19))
 (segment (start 134.62 105.41) (end 136.1443 105.41) (width 0.254) (layer B.Cu) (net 19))
 (segment (start 137.16 104.902) (end 136.2072 104.902) (width 0.254) (layer B.Cu) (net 19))
 (segment (start 143.4377 101.6723) (end 148.59 96.52) (width 0.254) (layer F.Cu) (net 19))
 (segment (start 133.7177 101.6723) (end 143.4377 101.6723) (width 0.254) (layer F.Cu) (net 19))
 (segment (start 133.0886 102.3014) (end 133.7177 101.6723) (width 0.254) (layer F.Cu) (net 19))
 (segment (start 133.0886 103.3673) (end 133.0886 102.3014) (width 0.254) (layer F.Cu) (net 19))
 (segment (start 133.9626 104.2413) (end 133.0886 103.3673) (width 0.254) (layer F.Cu) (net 19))
 (segment (start 134.62 104.2413) (end 133.9626 104.2413) (width 0.254) (layer F.Cu) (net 19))
 (segment (start 134.62 105.41) (end 134.62 104.2413) (width 0.254) (layer F.Cu) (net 19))
 (segment (start 144.78 102.87) (end 134.62 102.87) (width 0.254) (layer F.Cu) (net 20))
 (segment (start 148.59 99.06) (end 144.78 102.87) (width 0.254) (layer F.Cu) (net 20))
 (segment (start 121.92 113.03) (end 125.5 113.03) (width 0.254) (layer F.Cu) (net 14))
 (segment (start 129.33 111.76) (end 129.4824 111.9123) (width 0.254) (layer F.Cu) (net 3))
 (segment (start 147.5011 112.8489) (end 148.59 111.76) (width 0.254) (layer F.Cu) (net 3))
 (segment (start 130.419 112.8489) (end 147.5011 112.8489) (width 0.254) (layer F.Cu) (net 3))
 (segment (start 129.4824 111.9123) (end 130.419 112.8489) (width 0.254) (layer F.Cu) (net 3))
 (segment (start 134.62 100.33) (end 134.62 99.0343) (width 0.508) (layer F.Cu) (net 3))
 (segment (start 126.0905 99.0343) (end 128.6694 99.0343) (width 0.508) (layer F.Cu) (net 3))
 (segment (start 124.46 97.4038) (end 126.0905 99.0343) (width 0.508) (layer F.Cu) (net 3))
 (segment (start 124.46 96.73) (end 124.46 97.4038) (width 0.508) (layer F.Cu) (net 3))
 (segment (start 128.6694 99.0343) (end 134.62 99.0343) (width 0.508) (layer F.Cu) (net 3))
 (segment (start 128.6694 109.8806) (end 128.06 110.49) (width 0.508) (layer F.Cu) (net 3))
 (segment (start 128.6694 99.0343) (end 128.6694 109.8806) (width 0.508) (layer F.Cu) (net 3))
 (segment (start 125.5 110.49) (end 128.06 110.49) (width 0.508) (layer F.Cu) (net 3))
 (segment (start 128.06 110.49) (end 129.33 111.76) (width 0.508) (layer F.Cu) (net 3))
 (segment (start 124.77 96.73) (end 128.5 93) (width 0.508) (layer B.Cu) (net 3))
 (segment (start 124.46 96.73) (end 124.77 96.73) (width 0.508) (layer B.Cu) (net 3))
 (segment (start 135.89 92.71) (end 142.24 92.71) (width 0.508) (layer F.Cu) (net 1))
 (segment (start 142.24 92.71) (end 142.24 93.9168) (width 0.508) (layer B.Cu) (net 1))
 (segment (start 143.8156 111.4544) (end 143.51 111.76) (width 0.508) (layer B.Cu) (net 1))
 (segment (start 143.8156 95.1153) (end 143.8156 111.4544) (width 0.508) (layer B.Cu) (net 1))
 (segment (start 142.6171 93.9168) (end 143.8156 95.1153) (width 0.508) (layer B.Cu) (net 1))
 (segment (start 142.24 93.9168) (end 142.6171 93.9168) (width 0.508) (layer B.Cu) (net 1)))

